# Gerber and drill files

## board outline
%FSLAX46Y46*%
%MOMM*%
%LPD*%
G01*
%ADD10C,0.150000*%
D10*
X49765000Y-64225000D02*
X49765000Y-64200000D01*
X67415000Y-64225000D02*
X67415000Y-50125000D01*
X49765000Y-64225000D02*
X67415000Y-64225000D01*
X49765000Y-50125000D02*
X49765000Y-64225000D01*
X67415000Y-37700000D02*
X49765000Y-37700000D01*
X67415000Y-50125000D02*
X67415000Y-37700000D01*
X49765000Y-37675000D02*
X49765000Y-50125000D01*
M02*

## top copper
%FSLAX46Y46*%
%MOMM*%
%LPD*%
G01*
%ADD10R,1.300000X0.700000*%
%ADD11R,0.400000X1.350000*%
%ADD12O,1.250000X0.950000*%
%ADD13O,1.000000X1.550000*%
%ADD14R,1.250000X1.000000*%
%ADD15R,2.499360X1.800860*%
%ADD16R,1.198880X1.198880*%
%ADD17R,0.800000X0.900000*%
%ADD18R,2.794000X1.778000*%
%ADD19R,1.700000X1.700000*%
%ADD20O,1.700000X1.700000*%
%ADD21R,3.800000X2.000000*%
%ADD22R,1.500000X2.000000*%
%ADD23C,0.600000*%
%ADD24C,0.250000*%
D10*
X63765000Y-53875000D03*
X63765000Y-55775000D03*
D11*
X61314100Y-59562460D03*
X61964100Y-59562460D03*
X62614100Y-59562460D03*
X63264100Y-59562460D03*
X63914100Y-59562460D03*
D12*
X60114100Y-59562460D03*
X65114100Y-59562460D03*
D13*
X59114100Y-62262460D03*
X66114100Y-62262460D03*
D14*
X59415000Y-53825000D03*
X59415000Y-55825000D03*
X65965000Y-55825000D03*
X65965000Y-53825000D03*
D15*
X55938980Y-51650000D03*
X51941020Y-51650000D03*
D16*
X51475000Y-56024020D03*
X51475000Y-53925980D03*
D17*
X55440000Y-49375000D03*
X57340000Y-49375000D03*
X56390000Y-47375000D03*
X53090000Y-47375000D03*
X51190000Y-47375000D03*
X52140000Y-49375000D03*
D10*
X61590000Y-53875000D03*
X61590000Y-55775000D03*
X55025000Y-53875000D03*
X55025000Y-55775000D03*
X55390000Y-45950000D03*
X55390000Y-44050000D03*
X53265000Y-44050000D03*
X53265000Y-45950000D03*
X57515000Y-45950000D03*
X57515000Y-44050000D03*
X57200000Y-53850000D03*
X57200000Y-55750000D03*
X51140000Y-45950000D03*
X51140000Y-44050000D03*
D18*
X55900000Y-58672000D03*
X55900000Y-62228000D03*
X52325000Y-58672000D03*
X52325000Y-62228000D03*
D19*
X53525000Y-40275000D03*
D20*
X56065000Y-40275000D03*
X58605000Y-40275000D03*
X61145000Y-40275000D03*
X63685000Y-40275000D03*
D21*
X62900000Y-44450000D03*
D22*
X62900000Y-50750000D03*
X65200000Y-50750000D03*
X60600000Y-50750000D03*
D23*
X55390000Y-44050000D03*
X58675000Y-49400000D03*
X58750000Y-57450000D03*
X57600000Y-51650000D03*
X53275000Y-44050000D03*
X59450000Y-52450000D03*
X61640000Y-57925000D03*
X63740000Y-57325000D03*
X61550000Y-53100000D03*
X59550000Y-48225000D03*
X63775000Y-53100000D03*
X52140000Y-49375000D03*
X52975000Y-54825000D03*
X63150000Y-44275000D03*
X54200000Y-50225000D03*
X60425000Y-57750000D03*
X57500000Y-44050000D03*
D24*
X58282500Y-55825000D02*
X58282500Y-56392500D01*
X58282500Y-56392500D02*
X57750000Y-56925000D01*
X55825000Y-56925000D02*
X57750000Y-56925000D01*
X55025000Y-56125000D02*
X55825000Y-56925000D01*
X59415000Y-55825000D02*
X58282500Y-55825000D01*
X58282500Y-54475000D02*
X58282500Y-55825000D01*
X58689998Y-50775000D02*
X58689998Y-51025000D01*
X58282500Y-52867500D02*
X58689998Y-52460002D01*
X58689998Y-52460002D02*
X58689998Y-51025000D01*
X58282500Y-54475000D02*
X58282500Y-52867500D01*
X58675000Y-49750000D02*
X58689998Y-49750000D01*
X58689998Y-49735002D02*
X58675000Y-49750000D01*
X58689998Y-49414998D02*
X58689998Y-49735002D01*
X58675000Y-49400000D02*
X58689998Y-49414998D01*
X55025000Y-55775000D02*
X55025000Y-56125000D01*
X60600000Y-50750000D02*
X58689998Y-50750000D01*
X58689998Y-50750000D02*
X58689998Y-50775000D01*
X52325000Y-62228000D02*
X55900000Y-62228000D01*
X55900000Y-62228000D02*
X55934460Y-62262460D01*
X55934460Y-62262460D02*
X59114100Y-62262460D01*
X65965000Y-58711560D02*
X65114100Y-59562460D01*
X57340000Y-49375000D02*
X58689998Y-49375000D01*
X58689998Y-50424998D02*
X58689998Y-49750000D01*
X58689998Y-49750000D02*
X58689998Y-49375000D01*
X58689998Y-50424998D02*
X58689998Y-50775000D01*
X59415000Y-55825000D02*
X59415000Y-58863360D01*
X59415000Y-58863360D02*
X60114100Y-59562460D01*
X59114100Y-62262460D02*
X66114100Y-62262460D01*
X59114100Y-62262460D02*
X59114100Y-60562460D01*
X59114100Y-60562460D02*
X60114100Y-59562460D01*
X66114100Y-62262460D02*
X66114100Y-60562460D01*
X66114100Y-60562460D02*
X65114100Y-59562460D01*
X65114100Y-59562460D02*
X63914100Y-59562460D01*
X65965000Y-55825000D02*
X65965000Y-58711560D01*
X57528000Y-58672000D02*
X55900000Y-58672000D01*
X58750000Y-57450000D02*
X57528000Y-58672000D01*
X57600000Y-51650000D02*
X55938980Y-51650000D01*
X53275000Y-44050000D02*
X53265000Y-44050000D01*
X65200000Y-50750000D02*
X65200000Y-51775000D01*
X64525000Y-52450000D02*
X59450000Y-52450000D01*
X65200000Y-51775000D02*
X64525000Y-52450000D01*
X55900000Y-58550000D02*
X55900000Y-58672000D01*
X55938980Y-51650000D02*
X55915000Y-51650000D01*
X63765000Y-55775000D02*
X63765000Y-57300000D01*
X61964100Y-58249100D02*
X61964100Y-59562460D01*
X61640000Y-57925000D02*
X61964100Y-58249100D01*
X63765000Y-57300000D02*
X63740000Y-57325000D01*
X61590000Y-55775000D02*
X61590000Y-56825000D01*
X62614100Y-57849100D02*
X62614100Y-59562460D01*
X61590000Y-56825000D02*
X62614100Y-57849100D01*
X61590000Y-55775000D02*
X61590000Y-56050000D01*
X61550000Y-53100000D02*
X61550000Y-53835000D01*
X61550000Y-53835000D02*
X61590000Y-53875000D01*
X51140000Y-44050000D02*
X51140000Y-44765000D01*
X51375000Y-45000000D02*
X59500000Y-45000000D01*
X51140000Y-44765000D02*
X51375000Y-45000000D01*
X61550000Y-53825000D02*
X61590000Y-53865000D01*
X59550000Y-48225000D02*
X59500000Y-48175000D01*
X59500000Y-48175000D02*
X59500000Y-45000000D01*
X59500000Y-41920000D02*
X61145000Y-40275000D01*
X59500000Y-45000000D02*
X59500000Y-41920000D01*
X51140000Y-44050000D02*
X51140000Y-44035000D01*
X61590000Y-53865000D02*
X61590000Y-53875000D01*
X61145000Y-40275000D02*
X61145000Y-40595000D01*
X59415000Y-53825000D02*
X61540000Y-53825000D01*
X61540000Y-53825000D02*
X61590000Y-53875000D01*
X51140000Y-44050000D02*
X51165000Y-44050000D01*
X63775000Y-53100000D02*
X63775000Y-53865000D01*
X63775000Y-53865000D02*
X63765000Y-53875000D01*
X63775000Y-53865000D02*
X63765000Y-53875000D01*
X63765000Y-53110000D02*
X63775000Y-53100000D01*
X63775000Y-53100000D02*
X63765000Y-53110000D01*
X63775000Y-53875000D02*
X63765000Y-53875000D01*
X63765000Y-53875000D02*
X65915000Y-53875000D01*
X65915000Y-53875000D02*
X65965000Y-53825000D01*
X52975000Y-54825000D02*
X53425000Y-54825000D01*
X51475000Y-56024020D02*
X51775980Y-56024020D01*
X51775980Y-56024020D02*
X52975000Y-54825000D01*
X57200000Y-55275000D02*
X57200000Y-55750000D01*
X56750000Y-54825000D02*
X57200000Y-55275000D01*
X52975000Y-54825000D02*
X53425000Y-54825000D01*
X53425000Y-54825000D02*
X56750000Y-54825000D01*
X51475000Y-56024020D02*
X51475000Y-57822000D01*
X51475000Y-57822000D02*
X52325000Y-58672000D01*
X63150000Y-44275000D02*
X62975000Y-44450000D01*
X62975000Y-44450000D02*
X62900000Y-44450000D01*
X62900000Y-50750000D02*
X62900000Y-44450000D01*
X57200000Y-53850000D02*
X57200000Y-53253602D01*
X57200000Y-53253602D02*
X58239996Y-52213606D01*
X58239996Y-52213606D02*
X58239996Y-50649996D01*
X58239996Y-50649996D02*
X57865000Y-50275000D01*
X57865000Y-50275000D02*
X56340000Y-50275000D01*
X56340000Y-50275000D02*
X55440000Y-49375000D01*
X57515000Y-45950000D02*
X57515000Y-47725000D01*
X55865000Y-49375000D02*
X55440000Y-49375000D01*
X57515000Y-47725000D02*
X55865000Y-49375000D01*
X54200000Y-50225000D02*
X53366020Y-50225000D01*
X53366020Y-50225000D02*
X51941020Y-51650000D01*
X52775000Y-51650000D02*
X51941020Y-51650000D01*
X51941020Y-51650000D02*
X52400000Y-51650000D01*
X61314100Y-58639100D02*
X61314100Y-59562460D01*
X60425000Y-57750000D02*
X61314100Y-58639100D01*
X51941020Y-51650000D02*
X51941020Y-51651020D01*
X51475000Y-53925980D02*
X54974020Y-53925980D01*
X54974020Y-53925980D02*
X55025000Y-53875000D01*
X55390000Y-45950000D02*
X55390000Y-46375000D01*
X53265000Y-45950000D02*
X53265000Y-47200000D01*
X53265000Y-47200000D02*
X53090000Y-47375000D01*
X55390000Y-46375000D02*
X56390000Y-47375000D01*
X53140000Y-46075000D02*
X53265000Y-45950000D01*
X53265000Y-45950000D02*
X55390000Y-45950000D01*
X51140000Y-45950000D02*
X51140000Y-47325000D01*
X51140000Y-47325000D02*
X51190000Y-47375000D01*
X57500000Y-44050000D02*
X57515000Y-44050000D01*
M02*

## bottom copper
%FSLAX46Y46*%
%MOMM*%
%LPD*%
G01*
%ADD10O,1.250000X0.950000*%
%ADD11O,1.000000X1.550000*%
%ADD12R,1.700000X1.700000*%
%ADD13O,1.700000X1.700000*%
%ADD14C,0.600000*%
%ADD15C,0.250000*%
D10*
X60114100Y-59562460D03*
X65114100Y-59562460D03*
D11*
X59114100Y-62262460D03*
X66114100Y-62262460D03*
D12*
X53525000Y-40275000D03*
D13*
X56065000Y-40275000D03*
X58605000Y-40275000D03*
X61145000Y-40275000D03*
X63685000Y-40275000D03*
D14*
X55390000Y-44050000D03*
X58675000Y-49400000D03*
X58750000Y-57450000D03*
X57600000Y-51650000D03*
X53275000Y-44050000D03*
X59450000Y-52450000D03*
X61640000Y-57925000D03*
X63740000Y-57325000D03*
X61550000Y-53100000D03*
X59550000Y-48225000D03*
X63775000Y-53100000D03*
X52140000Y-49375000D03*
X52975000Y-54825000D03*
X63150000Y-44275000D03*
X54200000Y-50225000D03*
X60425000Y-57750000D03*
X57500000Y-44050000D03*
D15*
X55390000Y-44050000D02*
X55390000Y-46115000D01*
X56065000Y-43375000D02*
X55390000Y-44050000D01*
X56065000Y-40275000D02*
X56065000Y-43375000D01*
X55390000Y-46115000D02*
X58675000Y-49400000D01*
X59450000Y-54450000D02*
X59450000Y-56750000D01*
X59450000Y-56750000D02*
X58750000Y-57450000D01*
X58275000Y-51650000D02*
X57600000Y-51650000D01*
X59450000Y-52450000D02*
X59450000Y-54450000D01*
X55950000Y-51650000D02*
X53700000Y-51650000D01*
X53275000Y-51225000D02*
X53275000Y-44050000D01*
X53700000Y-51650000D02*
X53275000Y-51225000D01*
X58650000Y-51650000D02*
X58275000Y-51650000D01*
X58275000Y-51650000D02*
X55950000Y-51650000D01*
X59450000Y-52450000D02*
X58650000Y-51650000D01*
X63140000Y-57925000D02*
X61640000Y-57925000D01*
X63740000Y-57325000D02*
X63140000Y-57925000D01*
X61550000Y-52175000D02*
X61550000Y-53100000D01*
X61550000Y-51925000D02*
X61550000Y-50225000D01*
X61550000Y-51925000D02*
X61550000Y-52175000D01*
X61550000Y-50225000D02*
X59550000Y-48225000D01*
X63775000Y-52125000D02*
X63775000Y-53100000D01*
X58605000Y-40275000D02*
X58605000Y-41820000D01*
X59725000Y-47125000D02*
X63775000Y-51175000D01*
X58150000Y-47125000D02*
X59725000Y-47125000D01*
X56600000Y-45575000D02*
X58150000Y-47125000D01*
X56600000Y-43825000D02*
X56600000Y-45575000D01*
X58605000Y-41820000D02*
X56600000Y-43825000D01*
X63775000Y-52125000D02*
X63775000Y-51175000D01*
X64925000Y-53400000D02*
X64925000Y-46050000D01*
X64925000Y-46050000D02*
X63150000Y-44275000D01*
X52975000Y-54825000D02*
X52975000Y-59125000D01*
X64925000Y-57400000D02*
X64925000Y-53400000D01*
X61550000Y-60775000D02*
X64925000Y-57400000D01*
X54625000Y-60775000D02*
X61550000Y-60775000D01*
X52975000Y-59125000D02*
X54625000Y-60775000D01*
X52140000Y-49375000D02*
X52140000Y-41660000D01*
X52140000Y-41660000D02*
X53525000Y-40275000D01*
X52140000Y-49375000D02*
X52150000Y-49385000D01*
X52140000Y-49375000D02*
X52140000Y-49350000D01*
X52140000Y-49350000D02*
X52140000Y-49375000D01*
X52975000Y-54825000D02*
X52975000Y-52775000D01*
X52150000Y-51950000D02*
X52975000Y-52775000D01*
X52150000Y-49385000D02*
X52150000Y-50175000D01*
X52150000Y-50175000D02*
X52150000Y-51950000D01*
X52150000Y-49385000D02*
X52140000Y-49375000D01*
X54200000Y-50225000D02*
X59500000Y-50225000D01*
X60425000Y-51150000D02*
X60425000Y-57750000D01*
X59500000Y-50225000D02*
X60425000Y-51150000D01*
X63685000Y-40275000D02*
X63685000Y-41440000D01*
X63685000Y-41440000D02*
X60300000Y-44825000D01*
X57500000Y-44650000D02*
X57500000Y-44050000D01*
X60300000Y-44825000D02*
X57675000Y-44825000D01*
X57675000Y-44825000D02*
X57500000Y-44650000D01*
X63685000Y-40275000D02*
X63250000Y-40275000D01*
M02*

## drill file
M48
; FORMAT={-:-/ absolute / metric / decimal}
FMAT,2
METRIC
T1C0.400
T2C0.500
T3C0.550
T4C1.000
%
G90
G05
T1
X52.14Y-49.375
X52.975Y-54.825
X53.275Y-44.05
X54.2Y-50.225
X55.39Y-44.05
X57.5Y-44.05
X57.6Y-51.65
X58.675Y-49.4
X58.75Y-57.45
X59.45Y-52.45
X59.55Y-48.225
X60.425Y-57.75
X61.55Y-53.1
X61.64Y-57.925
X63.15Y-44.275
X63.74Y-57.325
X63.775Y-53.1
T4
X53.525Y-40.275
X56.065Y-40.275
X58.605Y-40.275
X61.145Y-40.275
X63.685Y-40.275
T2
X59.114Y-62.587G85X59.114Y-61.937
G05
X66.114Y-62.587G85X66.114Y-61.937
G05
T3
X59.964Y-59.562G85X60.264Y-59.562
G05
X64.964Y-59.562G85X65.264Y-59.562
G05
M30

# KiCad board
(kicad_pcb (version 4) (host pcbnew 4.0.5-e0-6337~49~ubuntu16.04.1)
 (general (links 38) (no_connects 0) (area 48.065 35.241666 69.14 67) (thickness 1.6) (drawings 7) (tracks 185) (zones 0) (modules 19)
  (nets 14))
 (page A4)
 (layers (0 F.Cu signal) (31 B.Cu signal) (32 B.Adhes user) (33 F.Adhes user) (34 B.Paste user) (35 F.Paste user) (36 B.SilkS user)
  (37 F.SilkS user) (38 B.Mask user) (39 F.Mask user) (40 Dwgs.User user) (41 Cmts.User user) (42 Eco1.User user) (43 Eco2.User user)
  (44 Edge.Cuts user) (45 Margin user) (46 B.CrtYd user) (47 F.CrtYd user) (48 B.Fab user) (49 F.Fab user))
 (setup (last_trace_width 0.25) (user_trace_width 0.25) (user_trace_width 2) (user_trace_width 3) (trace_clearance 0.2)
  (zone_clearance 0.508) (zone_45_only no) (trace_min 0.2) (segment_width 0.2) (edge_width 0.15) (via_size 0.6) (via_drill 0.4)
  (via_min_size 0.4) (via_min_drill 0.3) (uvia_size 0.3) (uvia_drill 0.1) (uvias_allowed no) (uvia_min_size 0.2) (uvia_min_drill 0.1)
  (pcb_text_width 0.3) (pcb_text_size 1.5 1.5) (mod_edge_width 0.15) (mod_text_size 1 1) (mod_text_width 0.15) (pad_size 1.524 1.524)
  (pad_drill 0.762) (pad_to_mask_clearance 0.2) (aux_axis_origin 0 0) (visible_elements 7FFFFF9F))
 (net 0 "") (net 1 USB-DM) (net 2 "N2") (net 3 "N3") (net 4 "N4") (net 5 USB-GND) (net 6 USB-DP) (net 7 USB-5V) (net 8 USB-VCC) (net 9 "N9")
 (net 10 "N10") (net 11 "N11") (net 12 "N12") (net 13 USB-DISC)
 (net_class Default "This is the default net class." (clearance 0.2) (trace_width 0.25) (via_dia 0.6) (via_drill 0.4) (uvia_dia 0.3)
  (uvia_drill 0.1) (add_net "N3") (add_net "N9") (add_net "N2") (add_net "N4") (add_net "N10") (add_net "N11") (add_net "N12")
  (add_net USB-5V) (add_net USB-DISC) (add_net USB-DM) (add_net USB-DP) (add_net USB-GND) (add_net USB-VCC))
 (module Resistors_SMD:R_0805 (layer F.Cu) (at 63.765 54.825 270)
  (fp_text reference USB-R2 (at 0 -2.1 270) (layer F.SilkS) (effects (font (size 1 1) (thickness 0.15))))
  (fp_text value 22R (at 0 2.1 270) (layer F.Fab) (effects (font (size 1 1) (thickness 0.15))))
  (pad 1 smd rect (at -0.95 0 270) (size 0.7 1.3) (layers F.Cu F.Paste F.Mask) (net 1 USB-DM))
  (pad 2 smd rect (at 0.95 0 270) (size 0.7 1.3) (layers F.Cu F.Paste F.Mask) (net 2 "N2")))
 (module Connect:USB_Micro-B (layer F.Cu) (at 62.615 61.125)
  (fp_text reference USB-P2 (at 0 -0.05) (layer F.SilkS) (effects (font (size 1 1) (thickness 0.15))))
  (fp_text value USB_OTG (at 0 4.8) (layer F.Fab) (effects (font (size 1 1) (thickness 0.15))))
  (pad 1 smd rect (at -1.3009 -1.56254 90) (size 1.35 0.4) (layers F.Cu F.Paste F.Mask) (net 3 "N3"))
  (pad 2 smd rect (at -0.6509 -1.56254 90) (size 1.35 0.4) (layers F.Cu F.Paste F.Mask) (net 2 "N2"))
  (pad 3 smd rect (at -0.0009 -1.56254 90) (size 1.35 0.4) (layers F.Cu F.Paste F.Mask) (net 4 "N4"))
  (pad 4 smd rect (at 0.6491 -1.56254 90) (size 1.35 0.4) (layers F.Cu F.Paste F.Mask))
  (pad 5 smd rect (at 1.2991 -1.56254 90) (size 1.35 0.4) (layers F.Cu F.Paste F.Mask) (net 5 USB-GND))
  (pad 6 thru_hole oval (at -2.5009 -1.56254 90) (size 0.95 1.25) (drill oval 0.55 0.85) (layers *.Cu *.Mask) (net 5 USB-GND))
  (pad 6 thru_hole oval (at 2.4991 -1.56254 90) (size 0.95 1.25) (drill oval 0.55 0.85) (layers *.Cu *.Mask) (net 5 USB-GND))
  (pad 6 thru_hole oval (at -3.5009 1.13746 90) (size 1.55 1) (drill oval 1.15 0.5) (layers *.Cu *.Mask) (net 5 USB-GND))
  (pad 6 thru_hole oval (at 3.4991 1.13746 90) (size 1.55 1) (drill oval 1.15 0.5) (layers *.Cu *.Mask) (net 5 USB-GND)))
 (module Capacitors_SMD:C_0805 (layer F.Cu) (at 59.415 54.825 270)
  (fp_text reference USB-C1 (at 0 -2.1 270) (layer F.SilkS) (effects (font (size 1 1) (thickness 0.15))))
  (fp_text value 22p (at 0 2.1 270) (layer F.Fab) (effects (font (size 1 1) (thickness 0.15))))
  (pad 1 smd rect (at -1 0 270) (size 1 1.25) (layers F.Cu F.Paste F.Mask) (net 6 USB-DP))
  (pad 2 smd rect (at 1 0 270) (size 1 1.25) (layers F.Cu F.Paste F.Mask) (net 5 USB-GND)))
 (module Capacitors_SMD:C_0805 (layer F.Cu) (at 65.965 54.825 90)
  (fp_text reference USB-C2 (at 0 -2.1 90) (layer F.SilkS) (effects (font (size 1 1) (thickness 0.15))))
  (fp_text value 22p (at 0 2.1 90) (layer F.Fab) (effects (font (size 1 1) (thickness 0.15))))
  (pad 1 smd rect (at -1 0 90) (size 1 1.25) (layers F.Cu F.Paste F.Mask) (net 5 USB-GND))
  (pad 2 smd rect (at 1 0 90) (size 1 1.25) (layers F.Cu F.Paste F.Mask) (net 1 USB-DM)))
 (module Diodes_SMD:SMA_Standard (layer F.Cu) (at 53.94 51.65 180)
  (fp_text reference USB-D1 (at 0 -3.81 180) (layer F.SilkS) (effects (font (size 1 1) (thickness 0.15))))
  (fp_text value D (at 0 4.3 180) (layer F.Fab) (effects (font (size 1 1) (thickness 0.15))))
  (pad 1 smd rect (at -1.99898 0 180) (size 2.49936 1.80086) (layers F.Cu F.Paste F.Mask) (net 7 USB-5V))
  (pad 2 smd rect (at 1.99898 0 180) (size 2.49936 1.80086) (layers F.Cu F.Paste F.Mask) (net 3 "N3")))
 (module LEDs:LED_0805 (layer F.Cu) (at 51.475 54.975 270)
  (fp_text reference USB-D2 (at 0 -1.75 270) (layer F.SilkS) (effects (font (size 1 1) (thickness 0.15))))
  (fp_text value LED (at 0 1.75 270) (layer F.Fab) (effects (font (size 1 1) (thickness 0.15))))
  (pad 2 smd rect (at 1.04902 0 90) (size 1.19888 1.19888) (layers F.Cu F.Paste F.Mask) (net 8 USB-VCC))
  (pad 1 smd rect (at -1.04902 0 90) (size 1.19888 1.19888) (layers F.Cu F.Paste F.Mask) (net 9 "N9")))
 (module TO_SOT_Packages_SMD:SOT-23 (layer F.Cu) (at 56.39 48.375 90)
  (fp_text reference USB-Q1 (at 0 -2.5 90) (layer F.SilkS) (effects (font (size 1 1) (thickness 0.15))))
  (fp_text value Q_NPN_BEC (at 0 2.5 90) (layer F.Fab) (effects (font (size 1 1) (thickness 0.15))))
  (pad 1 smd rect (at -1 -0.95 90) (size 0.9 0.8) (layers F.Cu F.Paste F.Mask) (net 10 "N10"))
  (pad 2 smd rect (at -1 0.95 90) (size 0.9 0.8) (layers F.Cu F.Paste F.Mask) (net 5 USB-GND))
  (pad 3 smd rect (at 1 0 90) (size 0.9 0.8) (layers F.Cu F.Paste F.Mask) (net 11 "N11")))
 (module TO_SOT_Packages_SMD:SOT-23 (layer F.Cu) (at 52.14 48.375 270)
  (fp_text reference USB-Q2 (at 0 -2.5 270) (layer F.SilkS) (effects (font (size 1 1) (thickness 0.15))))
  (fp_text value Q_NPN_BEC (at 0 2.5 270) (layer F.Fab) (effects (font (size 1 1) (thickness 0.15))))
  (pad 1 smd rect (at -1 -0.95 270) (size 0.9 0.8) (layers F.Cu F.Paste F.Mask) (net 11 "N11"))
  (pad 2 smd rect (at -1 0.95 270) (size 0.9 0.8) (layers F.Cu F.Paste F.Mask) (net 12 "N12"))
  (pad 3 smd rect (at 1 0 270) (size 0.9 0.8) (layers F.Cu F.Paste F.Mask) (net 8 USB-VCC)))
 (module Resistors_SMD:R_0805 (layer F.Cu) (at 61.59 54.825 270)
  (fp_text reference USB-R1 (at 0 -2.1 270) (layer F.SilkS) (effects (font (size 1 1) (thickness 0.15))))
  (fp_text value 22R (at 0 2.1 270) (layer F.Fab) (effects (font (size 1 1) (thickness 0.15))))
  (pad 1 smd rect (at -0.95 0 270) (size 0.7 1.3) (layers F.Cu F.Paste F.Mask) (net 6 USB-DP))
  (pad 2 smd rect (at 0.95 0 270) (size 0.7 1.3) (layers F.Cu F.Paste F.Mask) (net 4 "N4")))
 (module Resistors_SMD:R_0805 (layer F.Cu) (at 55.025 54.825 270)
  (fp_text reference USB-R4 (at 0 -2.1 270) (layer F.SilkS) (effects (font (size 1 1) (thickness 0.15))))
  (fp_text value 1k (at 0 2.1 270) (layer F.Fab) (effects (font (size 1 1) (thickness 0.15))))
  (pad 1 smd rect (at -0.95 0 270) (size 0.7 1.3) (layers F.Cu F.Paste F.Mask) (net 9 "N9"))
  (pad 2 smd rect (at 0.95 0 270) (size 0.7 1.3) (layers F.Cu F.Paste F.Mask) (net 5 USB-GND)))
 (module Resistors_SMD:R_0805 (layer F.Cu) (at 55.39 45 90)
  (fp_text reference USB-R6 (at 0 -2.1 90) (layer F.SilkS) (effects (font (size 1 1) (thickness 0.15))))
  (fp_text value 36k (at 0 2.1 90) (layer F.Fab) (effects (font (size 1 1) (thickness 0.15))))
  (pad 1 smd rect (at -0.95 0 90) (size 0.7 1.3) (layers F.Cu F.Paste F.Mask) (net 11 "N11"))
  (pad 2 smd rect (at 0.95 0 90) (size 0.7 1.3) (layers F.Cu F.Paste F.Mask) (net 5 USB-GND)))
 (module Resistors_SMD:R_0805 (layer F.Cu) (at 53.265 45 270)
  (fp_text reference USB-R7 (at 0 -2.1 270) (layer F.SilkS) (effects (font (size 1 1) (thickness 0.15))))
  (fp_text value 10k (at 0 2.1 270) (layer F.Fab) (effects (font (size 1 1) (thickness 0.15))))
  (pad 1 smd rect (at -0.95 0 270) (size 0.7 1.3) (layers F.Cu F.Paste F.Mask) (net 7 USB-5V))
  (pad 2 smd rect (at 0.95 0 270) (size 0.7 1.3) (layers F.Cu F.Paste F.Mask) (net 11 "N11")))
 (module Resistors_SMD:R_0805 (layer F.Cu) (at 57.515 45 90)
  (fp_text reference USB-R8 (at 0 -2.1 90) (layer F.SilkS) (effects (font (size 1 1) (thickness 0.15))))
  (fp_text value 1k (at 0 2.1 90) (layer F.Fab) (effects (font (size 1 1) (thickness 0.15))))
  (pad 1 smd rect (at -0.95 0 90) (size 0.7 1.3) (layers F.Cu F.Paste F.Mask) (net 10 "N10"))
  (pad 2 smd rect (at 0.95 0 90) (size 0.7 1.3) (layers F.Cu F.Paste F.Mask) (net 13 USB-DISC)))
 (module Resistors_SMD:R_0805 (layer F.Cu) (at 57.2 54.8 270)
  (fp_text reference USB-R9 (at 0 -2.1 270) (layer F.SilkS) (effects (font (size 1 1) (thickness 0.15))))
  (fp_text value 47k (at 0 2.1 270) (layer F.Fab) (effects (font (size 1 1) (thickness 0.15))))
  (pad 1 smd rect (at -0.95 0 270) (size 0.7 1.3) (layers F.Cu F.Paste F.Mask) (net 10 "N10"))
  (pad 2 smd rect (at 0.95 0 270) (size 0.7 1.3) (layers F.Cu F.Paste F.Mask) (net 8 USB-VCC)))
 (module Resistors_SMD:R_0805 (layer F.Cu) (at 51.14 45 90)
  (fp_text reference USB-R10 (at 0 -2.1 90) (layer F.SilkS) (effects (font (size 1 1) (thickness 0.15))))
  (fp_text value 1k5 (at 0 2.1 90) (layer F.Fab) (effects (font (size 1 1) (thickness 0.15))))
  (pad 1 smd rect (at -0.95 0 90) (size 0.7 1.3) (layers F.Cu F.Paste F.Mask) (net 12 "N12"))
  (pad 2 smd rect (at 0.95 0 90) (size 0.7 1.3) (layers F.Cu F.Paste F.Mask) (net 6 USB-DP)))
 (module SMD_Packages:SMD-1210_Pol (layer F.Cu) (at 55.9 60.45 270)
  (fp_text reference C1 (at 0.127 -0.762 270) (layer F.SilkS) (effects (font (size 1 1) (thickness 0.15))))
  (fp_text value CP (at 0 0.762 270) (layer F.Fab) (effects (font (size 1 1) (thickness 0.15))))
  (pad 1 smd rect (at -1.778 0 270) (size 1.778 2.794) (layers F.Cu F.Paste F.Mask) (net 7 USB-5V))
  (pad 2 smd rect (at 1.778 0 270) (size 1.778 2.794) (layers F.Cu F.Paste F.Mask) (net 5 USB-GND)))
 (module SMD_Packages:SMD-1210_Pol (layer F.Cu) (at 52.325 60.45 270)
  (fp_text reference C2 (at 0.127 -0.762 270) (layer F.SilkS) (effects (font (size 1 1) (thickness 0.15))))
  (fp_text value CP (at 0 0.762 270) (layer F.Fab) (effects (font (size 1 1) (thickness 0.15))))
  (pad 1 smd rect (at -1.778 0 270) (size 1.778 2.794) (layers F.Cu F.Paste F.Mask) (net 8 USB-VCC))
  (pad 2 smd rect (at 1.778 0 270) (size 1.778 2.794) (layers F.Cu F.Paste F.Mask) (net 5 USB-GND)))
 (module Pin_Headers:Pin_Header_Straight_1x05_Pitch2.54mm (layer F.Cu) (at 53.525 40.275 90)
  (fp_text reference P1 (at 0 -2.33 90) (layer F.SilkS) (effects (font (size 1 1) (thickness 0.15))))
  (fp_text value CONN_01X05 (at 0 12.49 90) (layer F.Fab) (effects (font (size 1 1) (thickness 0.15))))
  (pad 1 thru_hole rect (at 0 0 90) (size 1.7 1.7) (drill 1) (layers *.Cu *.Mask) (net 8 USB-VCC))
  (pad 2 thru_hole oval (at 0 2.54 90) (size 1.7 1.7) (drill 1) (layers *.Cu *.Mask) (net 5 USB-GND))
  (pad 3 thru_hole oval (at 0 5.08 90) (size 1.7 1.7) (drill 1) (layers *.Cu *.Mask) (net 1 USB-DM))
  (pad 4 thru_hole oval (at 0 7.62 90) (size 1.7 1.7) (drill 1) (layers *.Cu *.Mask) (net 6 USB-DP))
  (pad 5 thru_hole oval (at 0 10.16 90) (size 1.7 1.7) (drill 1) (layers *.Cu *.Mask) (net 13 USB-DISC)))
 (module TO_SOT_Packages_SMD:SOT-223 (layer F.Cu) (at 62.9 47.6 90)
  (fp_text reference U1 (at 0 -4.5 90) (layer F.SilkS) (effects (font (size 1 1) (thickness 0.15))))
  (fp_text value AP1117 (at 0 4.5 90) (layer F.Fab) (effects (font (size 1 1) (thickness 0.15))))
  (pad 4 smd rect (at 3.15 0 90) (size 2 3.8) (layers F.Cu F.Paste F.Mask) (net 8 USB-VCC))
  (pad 2 smd rect (at -3.15 0 90) (size 2 1.5) (layers F.Cu F.Paste F.Mask) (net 8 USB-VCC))
  (pad 3 smd rect (at -3.15 2.3 90) (size 2 1.5) (layers F.Cu F.Paste F.Mask) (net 7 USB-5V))
  (pad 1 smd rect (at -3.15 -2.3 90) (size 2 1.5) (layers F.Cu F.Paste F.Mask) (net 5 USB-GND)))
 (gr_line (start 49.765 64.225) (end 49.765 64.2) (angle 90) (layer Edge.Cuts) (width 0.15))
 (gr_line (start 67.415 64.225) (end 67.415 50.125) (angle 90) (layer Edge.Cuts) (width 0.15))
 (gr_line (start 49.765 64.225) (end 67.415 64.225) (angle 90) (layer Edge.Cuts) (width 0.15))
 (gr_line (start 49.765 50.125) (end 49.765 64.225) (angle 90) (layer Edge.Cuts) (width 0.15))
 (gr_line (start 67.415 37.7) (end 49.765 37.7) (angle 90) (layer Edge.Cuts) (width 0.15))
 (gr_line (start 67.415 50.125) (end 67.415 37.7) (angle 90) (layer Edge.Cuts) (width 0.15))
 (gr_line (start 49.765 37.675) (end 49.765 50.125) (angle 90) (layer Edge.Cuts) (width 0.15))
 (segment (start 58.2825 55.825) (end 58.2825 56.3925) (width 0.25) (layer F.Cu) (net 5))
 (segment (start 58.2825 56.3925) (end 57.75 56.925) (width 0.25) (layer F.Cu) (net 5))
 (segment (start 55.825 56.925) (end 57.75 56.925) (width 0.25) (layer F.Cu) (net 5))
 (segment (start 55.025 56.125) (end 55.825 56.925) (width 0.25) (layer F.Cu) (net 5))
 (segment (start 59.415 55.825) (end 58.2825 55.825) (width 0.25) (layer F.Cu) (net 5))
 (segment (start 58.2825 54.475) (end 58.2825 55.825) (width 0.25) (layer F.Cu) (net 5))
 (segment (start 58.689998 50.775) (end 58.689998 51.025) (width 0.25) (layer F.Cu) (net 5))
 (segment (start 58.2825 52.8675) (end 58.689998 52.460002) (width 0.25) (layer F.Cu) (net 5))
 (segment (start 58.689998 52.460002) (end 58.689998 51.025) (width 0.25) (layer F.Cu) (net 5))
 (segment (start 58.2825 54.475) (end 58.2825 52.8675) (width 0.25) (layer F.Cu) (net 5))
 (segment (start 55.39 44.05) (end 55.39 46.115) (width 0.25) (layer B.Cu) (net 5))
 (segment (start 56.065 43.375) (end 55.39 44.05) (width 0.25) (layer B.Cu) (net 5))
 (segment (start 56.065 40.275) (end 56.065 43.375) (width 0.25) (layer B.Cu) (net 5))
 (via (at 55.39 44.05) (size 0.6) (drill 0.4) (layers F.Cu B.Cu) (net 5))
 (segment (start 58.675 49.75) (end 58.689998 49.75) (width 0.25) (layer F.Cu) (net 5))
 (segment (start 58.689998 49.735002) (end 58.675 49.75) (width 0.25) (layer F.Cu) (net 5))
 (segment (start 58.689998 49.414998) (end 58.689998 49.735002) (width 0.25) (layer F.Cu) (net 5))
 (segment (start 58.675 49.4) (end 58.689998 49.414998) (width 0.25) (layer F.Cu) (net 5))
 (via (at 58.675 49.4) (size 0.6) (drill 0.4) (layers F.Cu B.Cu) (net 5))
 (segment (start 55.39 46.115) (end 58.675 49.4) (width 0.25) (layer B.Cu) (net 5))
 (segment (start 55.025 55.775) (end 55.025 56.125) (width 0.25) (layer F.Cu) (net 5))
 (segment (start 60.6 50.75) (end 58.689998 50.75) (width 0.25) (layer F.Cu) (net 5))
 (segment (start 58.689998 50.75) (end 58.689998 50.775) (width 0.25) (layer F.Cu) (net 5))
 (segment (start 52.325 62.228) (end 55.9 62.228) (width 0.25) (layer F.Cu) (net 5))
 (segment (start 55.9 62.228) (end 55.93446 62.26246) (width 0.25) (layer F.Cu) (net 5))
 (segment (start 55.93446 62.26246) (end 59.1141 62.26246) (width 0.25) (layer F.Cu) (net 5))
 (segment (start 65.965 58.71156) (end 65.1141 59.56246) (width 0.25) (layer F.Cu) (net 5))
 (segment (start 57.34 49.375) (end 58.689998 49.375) (width 0.25) (layer F.Cu) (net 5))
 (segment (start 58.689998 50.424998) (end 58.689998 49.75) (width 0.25) (layer F.Cu) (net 5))
 (segment (start 58.689998 49.75) (end 58.689998 49.375) (width 0.25) (layer F.Cu) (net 5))
 (segment (start 58.689998 50.424998) (end 58.689998 50.775) (width 0.25) (layer F.Cu) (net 5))
 (segment (start 59.415 55.825) (end 59.415 58.86336) (width 0.25) (layer F.Cu) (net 5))
 (segment (start 59.415 58.86336) (end 60.1141 59.56246) (width 0.25) (layer F.Cu) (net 5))
 (segment (start 59.1141 62.26246) (end 66.1141 62.26246) (width 0.25) (layer F.Cu) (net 5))
 (segment (start 59.1141 62.26246) (end 59.1141 60.56246) (width 0.25) (layer F.Cu) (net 5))
 (segment (start 59.1141 60.56246) (end 60.1141 59.56246) (width 0.25) (layer F.Cu) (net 5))
 (segment (start 66.1141 62.26246) (end 66.1141 60.56246) (width 0.25) (layer F.Cu) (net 5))
 (segment (start 66.1141 60.56246) (end 65.1141 59.56246) (width 0.25) (layer F.Cu) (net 5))
 (segment (start 65.1141 59.56246) (end 63.9141 59.56246) (width 0.25) (layer F.Cu) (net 5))
 (segment (start 65.965 55.825) (end 65.965 58.71156) (width 0.25) (layer F.Cu) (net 5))
 (segment (start 59.45 54.45) (end 59.45 56.75) (width 0.25) (layer B.Cu) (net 7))
 (segment (start 57.528 58.672) (end 55.9 58.672) (width 0.25) (layer F.Cu) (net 7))
 (segment (start 58.75 57.45) (end 57.528 58.672) (width 0.25) (layer F.Cu) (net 7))
 (via (at 58.75 57.45) (size 0.6) (drill 0.4) (layers F.Cu B.Cu) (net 7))
 (segment (start 59.45 56.75) (end 58.75 57.45) (width 0.25) (layer B.Cu) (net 7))
 (segment (start 58.275 51.65) (end 57.6 51.65) (width 0.25) (layer B.Cu) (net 7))
 (segment (start 57.6 51.65) (end 55.93898 51.65) (width 0.25) (layer F.Cu) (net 7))
 (via (at 57.6 51.65) (size 0.6) (drill 0.4) (layers F.Cu B.Cu) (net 7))
 (segment (start 59.45 52.45) (end 59.45 54.45) (width 0.25) (layer B.Cu) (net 7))
 (segment (start 55.95 51.65) (end 53.7 51.65) (width 0.25) (layer B.Cu) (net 7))
 (segment (start 53.275 44.05) (end 53.265 44.05) (width 0.25) (layer F.Cu) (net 7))
 (via (at 53.275 44.05) (size 0.6) (drill 0.4) (layers F.Cu B.Cu) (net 7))
 (segment (start 53.275 51.225) (end 53.275 44.05) (width 0.25) (layer B.Cu) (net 7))
 (segment (start 53.7 51.65) (end 53.275 51.225) (width 0.25) (layer B.Cu) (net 7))
 (segment (start 65.2 50.75) (end 65.2 51.775) (width 0.25) (layer F.Cu) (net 7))
 (segment (start 58.65 51.65) (end 58.275 51.65) (width 0.25) (layer B.Cu) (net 7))
 (segment (start 58.275 51.65) (end 55.95 51.65) (width 0.25) (layer B.Cu) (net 7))
 (segment (start 59.45 52.45) (end 58.65 51.65) (width 0.25) (layer B.Cu) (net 7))
 (via (at 59.45 52.45) (size 0.6) (drill 0.4) (layers F.Cu B.Cu) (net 7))
 (segment (start 64.525 52.45) (end 59.45 52.45) (width 0.25) (layer F.Cu) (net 7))
 (segment (start 65.2 51.775) (end 64.525 52.45) (width 0.25) (layer F.Cu) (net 7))
 (segment (start 55.9 58.55) (end 55.9 58.672) (width 0.25) (layer F.Cu) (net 7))
 (segment (start 55.93898 51.65) (end 55.915 51.65) (width 0.25) (layer F.Cu) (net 7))
 (segment (start 63.765 55.775) (end 63.765 57.3) (width 0.25) (layer F.Cu) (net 2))
 (segment (start 61.9641 58.2491) (end 61.9641 59.56246) (width 0.25) (layer F.Cu) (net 2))
 (segment (start 61.64 57.925) (end 61.9641 58.2491) (width 0.25) (layer F.Cu) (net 2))
 (via (at 61.64 57.925) (size 0.6) (drill 0.4) (layers F.Cu B.Cu) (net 2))
 (segment (start 63.14 57.925) (end 61.64 57.925) (width 0.25) (layer B.Cu) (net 2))
 (via (at 63.74 57.325) (size 0.6) (drill 0.4) (layers F.Cu B.Cu) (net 2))
 (segment (start 63.765 57.3) (end 63.74 57.325) (width 0.25) (layer F.Cu) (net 2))
 (segment (start 63.74 57.325) (end 63.14 57.925) (width 0.25) (layer B.Cu) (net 2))
 (segment (start 61.59 55.775) (end 61.59 56.825) (width 0.25) (layer F.Cu) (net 4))
 (segment (start 62.6141 57.8491) (end 62.6141 59.56246) (width 0.25) (layer F.Cu) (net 4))
 (segment (start 61.59 56.825) (end 62.6141 57.8491) (width 0.25) (layer F.Cu) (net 4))
 (segment (start 61.59 55.775) (end 61.59 56.05) (width 0.25) (layer F.Cu) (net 4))
 (segment (start 61.55 53.1) (end 61.55 53.835) (width 0.25) (layer F.Cu) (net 6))
 (segment (start 61.55 53.835) (end 61.59 53.875) (width 0.25) (layer F.Cu) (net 6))
 (segment (start 61.55 52.175) (end 61.55 53.1) (width 0.25) (layer B.Cu) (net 6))
 (via (at 61.55 53.1) (size 0.6) (drill 0.4) (layers F.Cu B.Cu) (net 6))
 (segment (start 51.14 44.05) (end 51.14 44.765) (width 0.25) (layer F.Cu) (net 6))
 (segment (start 51.375 45) (end 59.5 45) (width 0.25) (layer F.Cu) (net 6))
 (segment (start 51.14 44.765) (end 51.375 45) (width 0.25) (layer F.Cu) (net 6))
 (segment (start 61.55 51.925) (end 61.55 50.225) (width 0.25) (layer B.Cu) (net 6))
 (segment (start 61.55 51.925) (end 61.55 52.175) (width 0.25) (layer B.Cu) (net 6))
 (segment (start 61.55 53.825) (end 61.59 53.865) (width 0.25) (layer F.Cu) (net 6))
 (segment (start 61.55 50.225) (end 59.55 48.225) (width 0.25) (layer B.Cu) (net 6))
 (via (at 59.55 48.225) (size 0.6) (drill 0.4) (layers F.Cu B.Cu) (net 6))
 (segment (start 59.55 48.225) (end 59.5 48.175) (width 0.25) (layer F.Cu) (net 6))
 (segment (start 59.5 48.175) (end 59.5 45) (width 0.25) (layer F.Cu) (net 6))
 (segment (start 59.5 41.92) (end 61.145 40.275) (width 0.25) (layer F.Cu) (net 6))
 (segment (start 59.5 45) (end 59.5 41.92) (width 0.25) (layer F.Cu) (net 6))
 (segment (start 51.14 44.05) (end 51.14 44.035) (width 0.25) (layer F.Cu) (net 6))
 (segment (start 61.59 53.865) (end 61.59 53.875) (width 0.25) (layer F.Cu) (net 6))
 (segment (start 61.145 40.275) (end 61.145 40.595) (width 0.25) (layer F.Cu) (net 6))
 (segment (start 59.415 53.825) (end 61.54 53.825) (width 0.25) (layer F.Cu) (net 6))
 (segment (start 61.54 53.825) (end 61.59 53.875) (width 0.25) (layer F.Cu) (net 6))
 (segment (start 51.14 44.05) (end 51.165 44.05) (width 0.25) (layer F.Cu) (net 6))
 (segment (start 63.775 53.1) (end 63.775 53.865) (width 0.25) (layer F.Cu) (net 1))
 (segment (start 63.775 53.865) (end 63.765 53.875) (width 0.25) (layer F.Cu) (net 1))
 (segment (start 63.775 53.865) (end 63.765 53.875) (width 0.25) (layer F.Cu) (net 1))
 (segment (start 63.765 53.11) (end 63.775 53.1) (width 0.25) (layer F.Cu) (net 1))
 (segment (start 63.775 52.125) (end 63.775 53.1) (width 0.25) (layer B.Cu) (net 1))
 (segment (start 63.775 53.1) (end 63.765 53.11) (width 0.25) (layer F.Cu) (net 1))
 (via (at 63.775 53.1) (size 0.6) (drill 0.4) (layers F.Cu B.Cu) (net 1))
 (segment (start 58.605 40.275) (end 58.605 41.82) (width 0.25) (layer B.Cu) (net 1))
 (segment (start 59.725 47.125) (end 63.775 51.175) (width 0.25) (layer B.Cu) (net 1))
 (segment (start 58.15 47.125) (end 59.725 47.125) (width 0.25) (layer B.Cu) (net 1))
 (segment (start 56.6 45.575) (end 58.15 47.125) (width 0.25) (layer B.Cu) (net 1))
 (segment (start 56.6 43.825) (end 56.6 45.575) (width 0.25) (layer B.Cu) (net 1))
 (segment (start 58.605 41.82) (end 56.6 43.825) (width 0.25) (layer B.Cu) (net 1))
 (segment (start 63.775 52.125) (end 63.775 51.175) (width 0.25) (layer B.Cu) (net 1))
 (segment (start 63.775 53.875) (end 63.765 53.875) (width 0.25) (layer F.Cu) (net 1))
 (segment (start 63.765 53.875) (end 65.915 53.875) (width 0.25) (layer F.Cu) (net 1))
 (segment (start 65.915 53.875) (end 65.965 53.825) (width 0.25) (layer F.Cu) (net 1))
 (segment (start 64.925 53.4) (end 64.925 46.05) (width 0.25) (layer B.Cu) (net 8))
 (segment (start 64.925 46.05) (end 63.15 44.275) (width 0.25) (layer B.Cu) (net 8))
 (segment (start 52.975 54.825) (end 52.975 59.125) (width 0.25) (layer B.Cu) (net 8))
 (segment (start 64.925 57.4) (end 64.925 53.4) (width 0.25) (layer B.Cu) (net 8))
 (segment (start 61.55 60.775) (end 64.925 57.4) (width 0.25) (layer B.Cu) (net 8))
 (segment (start 54.625 60.775) (end 61.55 60.775) (width 0.25) (layer B.Cu) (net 8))
 (segment (start 52.975 59.125) (end 54.625 60.775) (width 0.25) (layer B.Cu) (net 8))
 (segment (start 52.14 49.375) (end 52.14 41.66) (width 0.25) (layer B.Cu) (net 8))
 (via (at 52.14 49.375) (size 0.6) (drill 0.4) (layers F.Cu B.Cu) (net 8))
 (segment (start 52.14 41.66) (end 53.525 40.275) (width 0.25) (layer B.Cu) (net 8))
 (segment (start 52.14 49.375) (end 52.15 49.385) (width 0.25) (layer B.Cu) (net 8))
 (segment (start 52.14 49.375) (end 52.14 49.35) (width 0.25) (layer B.Cu) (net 8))
 (segment (start 52.14 49.35) (end 52.14 49.375) (width 0.25) (layer B.Cu) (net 8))
 (via (at 52.975 54.825) (size 0.6) (drill 0.4) (layers F.Cu B.Cu) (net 8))
 (segment (start 52.975 54.825) (end 52.975 52.775) (width 0.25) (layer B.Cu) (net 8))
 (segment (start 52.15 51.95) (end 52.975 52.775) (width 0.25) (layer B.Cu) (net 8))
 (segment (start 52.15 49.385) (end 52.15 50.175) (width 0.25) (layer B.Cu) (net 8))
 (segment (start 52.15 50.175) (end 52.15 51.95) (width 0.25) (layer B.Cu) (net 8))
 (segment (start 52.15 49.385) (end 52.14 49.375) (width 0.25) (layer B.Cu) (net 8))
 (segment (start 52.975 54.825) (end 53.425 54.825) (width 0.25) (layer F.Cu) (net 8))
 (segment (start 51.475 56.02402) (end 51.77598 56.02402) (width 0.25) (layer F.Cu) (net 8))
 (segment (start 51.77598 56.02402) (end 52.975 54.825) (width 0.25) (layer F.Cu) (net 8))
 (segment (start 57.2 55.275) (end 57.2 55.75) (width 0.25) (layer F.Cu) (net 8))
 (segment (start 56.75 54.825) (end 57.2 55.275) (width 0.25) (layer F.Cu) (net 8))
 (segment (start 52.975 54.825) (end 53.425 54.825) (width 0.25) (layer F.Cu) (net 8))
 (segment (start 53.425 54.825) (end 56.75 54.825) (width 0.25) (layer F.Cu) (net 8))
 (segment (start 51.475 56.02402) (end 51.475 57.822) (width 0.25) (layer F.Cu) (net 8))
 (segment (start 51.475 57.822) (end 52.325 58.672) (width 0.25) (layer F.Cu) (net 8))
 (segment (start 63.15 44.275) (end 62.975 44.45) (width 0.25) (layer F.Cu) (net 8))
 (via (at 63.15 44.275) (size 0.6) (drill 0.4) (layers F.Cu B.Cu) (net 8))
 (segment (start 62.975 44.45) (end 62.9 44.45) (width 0.25) (layer F.Cu) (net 8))
 (segment (start 62.9 50.75) (end 62.9 44.45) (width 0.25) (layer F.Cu) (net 8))
 (segment (start 57.2 53.85) (end 57.2 53.253602) (width 0.25) (layer F.Cu) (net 10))
 (segment (start 57.2 53.253602) (end 58.239996 52.213606) (width 0.25) (layer F.Cu) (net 10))
 (segment (start 58.239996 52.213606) (end 58.239996 50.649996) (width 0.25) (layer F.Cu) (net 10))
 (segment (start 58.239996 50.649996) (end 57.865 50.275) (width 0.25) (layer F.Cu) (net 10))
 (segment (start 57.865 50.275) (end 56.34 50.275) (width 0.25) (layer F.Cu) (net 10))
 (segment (start 56.34 50.275) (end 55.44 49.375) (width 0.25) (layer F.Cu) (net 10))
 (segment (start 57.515 45.95) (end 57.515 47.725) (width 0.25) (layer F.Cu) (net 10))
 (segment (start 55.865 49.375) (end 55.44 49.375) (width 0.25) (layer F.Cu) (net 10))
 (segment (start 57.515 47.725) (end 55.865 49.375) (width 0.25) (layer F.Cu) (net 10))
 (segment (start 54.2 50.225) (end 59.5 50.225) (width 0.25) (layer B.Cu) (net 3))
 (segment (start 60.425 51.15) (end 60.425 57.75) (width 0.25) (layer B.Cu) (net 3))
 (segment (start 59.5 50.225) (end 60.425 51.15) (width 0.25) (layer B.Cu) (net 3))
 (segment (start 54.2 50.225) (end 53.36602 50.225) (width 0.25) (layer F.Cu) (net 3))
 (segment (start 53.36602 50.225) (end 51.94102 51.65) (width 0.25) (layer F.Cu) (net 3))
 (via (at 54.2 50.225) (size 0.6) (drill 0.4) (layers F.Cu B.Cu) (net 3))
 (segment (start 52.775 51.65) (end 51.94102 51.65) (width 0.25) (layer F.Cu) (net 3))
 (segment (start 51.94102 51.65) (end 52.4 51.65) (width 0.25) (layer F.Cu) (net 3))
 (segment (start 61.3141 58.6391) (end 61.3141 59.56246) (width 0.25) (layer F.Cu) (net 3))
 (via (at 60.425 57.75) (size 0.6) (drill 0.4) (layers F.Cu B.Cu) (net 3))
 (segment (start 60.425 57.75) (end 61.3141 58.6391) (width 0.25) (layer F.Cu) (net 3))
 (segment (start 51.94102 51.65) (end 51.94102 51.65102) (width 0.25) (layer F.Cu) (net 3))
 (segment (start 51.475 53.92598) (end 54.97402 53.92598) (width 0.25) (layer F.Cu) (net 9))
 (segment (start 54.97402 53.92598) (end 55.025 53.875) (width 0.25) (layer F.Cu) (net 9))
 (segment (start 55.39 45.95) (end 55.39 46.375) (width 0.25) (layer F.Cu) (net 11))
 (segment (start 53.265 45.95) (end 53.265 47.2) (width 0.25) (layer F.Cu) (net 11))
 (segment (start 53.265 47.2) (end 53.09 47.375) (width 0.25) (layer F.Cu) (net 11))
 (segment (start 55.39 46.375) (end 56.39 47.375) (width 0.25) (layer F.Cu) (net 11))
 (segment (start 53.14 46.075) (end 53.265 45.95) (width 0.25) (layer F.Cu) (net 11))
 (segment (start 53.265 45.95) (end 55.39 45.95) (width 0.25) (layer F.Cu) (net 11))
 (segment (start 51.14 45.95) (end 51.14 47.325) (width 0.25) (layer F.Cu) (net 12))
 (segment (start 51.14 47.325) (end 51.19 47.375) (width 0.25) (layer F.Cu) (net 12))
 (segment (start 63.685 40.275) (end 63.685 41.44) (width 0.25) (layer B.Cu) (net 13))
 (segment (start 63.685 41.44) (end 60.3 44.825) (width 0.25) (layer B.Cu) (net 13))
 (segment (start 57.5 44.65) (end 57.5 44.05) (width 0.25) (layer B.Cu) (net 13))
 (segment (start 57.5 44.05) (end 57.515 44.05) (width 0.25) (layer F.Cu) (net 13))
 (via (at 57.5 44.05) (size 0.6) (drill 0.4) (layers F.Cu B.Cu) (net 13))
 (segment (start 60.3 44.825) (end 57.675 44.825) (width 0.25) (layer B.Cu) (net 13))
 (segment (start 57.675 44.825) (end 57.5 44.65) (width 0.25) (layer B.Cu) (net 13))
 (segment (start 63.685 40.275) (end 63.25 40.275) (width 0.25) (layer B.Cu) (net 13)))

